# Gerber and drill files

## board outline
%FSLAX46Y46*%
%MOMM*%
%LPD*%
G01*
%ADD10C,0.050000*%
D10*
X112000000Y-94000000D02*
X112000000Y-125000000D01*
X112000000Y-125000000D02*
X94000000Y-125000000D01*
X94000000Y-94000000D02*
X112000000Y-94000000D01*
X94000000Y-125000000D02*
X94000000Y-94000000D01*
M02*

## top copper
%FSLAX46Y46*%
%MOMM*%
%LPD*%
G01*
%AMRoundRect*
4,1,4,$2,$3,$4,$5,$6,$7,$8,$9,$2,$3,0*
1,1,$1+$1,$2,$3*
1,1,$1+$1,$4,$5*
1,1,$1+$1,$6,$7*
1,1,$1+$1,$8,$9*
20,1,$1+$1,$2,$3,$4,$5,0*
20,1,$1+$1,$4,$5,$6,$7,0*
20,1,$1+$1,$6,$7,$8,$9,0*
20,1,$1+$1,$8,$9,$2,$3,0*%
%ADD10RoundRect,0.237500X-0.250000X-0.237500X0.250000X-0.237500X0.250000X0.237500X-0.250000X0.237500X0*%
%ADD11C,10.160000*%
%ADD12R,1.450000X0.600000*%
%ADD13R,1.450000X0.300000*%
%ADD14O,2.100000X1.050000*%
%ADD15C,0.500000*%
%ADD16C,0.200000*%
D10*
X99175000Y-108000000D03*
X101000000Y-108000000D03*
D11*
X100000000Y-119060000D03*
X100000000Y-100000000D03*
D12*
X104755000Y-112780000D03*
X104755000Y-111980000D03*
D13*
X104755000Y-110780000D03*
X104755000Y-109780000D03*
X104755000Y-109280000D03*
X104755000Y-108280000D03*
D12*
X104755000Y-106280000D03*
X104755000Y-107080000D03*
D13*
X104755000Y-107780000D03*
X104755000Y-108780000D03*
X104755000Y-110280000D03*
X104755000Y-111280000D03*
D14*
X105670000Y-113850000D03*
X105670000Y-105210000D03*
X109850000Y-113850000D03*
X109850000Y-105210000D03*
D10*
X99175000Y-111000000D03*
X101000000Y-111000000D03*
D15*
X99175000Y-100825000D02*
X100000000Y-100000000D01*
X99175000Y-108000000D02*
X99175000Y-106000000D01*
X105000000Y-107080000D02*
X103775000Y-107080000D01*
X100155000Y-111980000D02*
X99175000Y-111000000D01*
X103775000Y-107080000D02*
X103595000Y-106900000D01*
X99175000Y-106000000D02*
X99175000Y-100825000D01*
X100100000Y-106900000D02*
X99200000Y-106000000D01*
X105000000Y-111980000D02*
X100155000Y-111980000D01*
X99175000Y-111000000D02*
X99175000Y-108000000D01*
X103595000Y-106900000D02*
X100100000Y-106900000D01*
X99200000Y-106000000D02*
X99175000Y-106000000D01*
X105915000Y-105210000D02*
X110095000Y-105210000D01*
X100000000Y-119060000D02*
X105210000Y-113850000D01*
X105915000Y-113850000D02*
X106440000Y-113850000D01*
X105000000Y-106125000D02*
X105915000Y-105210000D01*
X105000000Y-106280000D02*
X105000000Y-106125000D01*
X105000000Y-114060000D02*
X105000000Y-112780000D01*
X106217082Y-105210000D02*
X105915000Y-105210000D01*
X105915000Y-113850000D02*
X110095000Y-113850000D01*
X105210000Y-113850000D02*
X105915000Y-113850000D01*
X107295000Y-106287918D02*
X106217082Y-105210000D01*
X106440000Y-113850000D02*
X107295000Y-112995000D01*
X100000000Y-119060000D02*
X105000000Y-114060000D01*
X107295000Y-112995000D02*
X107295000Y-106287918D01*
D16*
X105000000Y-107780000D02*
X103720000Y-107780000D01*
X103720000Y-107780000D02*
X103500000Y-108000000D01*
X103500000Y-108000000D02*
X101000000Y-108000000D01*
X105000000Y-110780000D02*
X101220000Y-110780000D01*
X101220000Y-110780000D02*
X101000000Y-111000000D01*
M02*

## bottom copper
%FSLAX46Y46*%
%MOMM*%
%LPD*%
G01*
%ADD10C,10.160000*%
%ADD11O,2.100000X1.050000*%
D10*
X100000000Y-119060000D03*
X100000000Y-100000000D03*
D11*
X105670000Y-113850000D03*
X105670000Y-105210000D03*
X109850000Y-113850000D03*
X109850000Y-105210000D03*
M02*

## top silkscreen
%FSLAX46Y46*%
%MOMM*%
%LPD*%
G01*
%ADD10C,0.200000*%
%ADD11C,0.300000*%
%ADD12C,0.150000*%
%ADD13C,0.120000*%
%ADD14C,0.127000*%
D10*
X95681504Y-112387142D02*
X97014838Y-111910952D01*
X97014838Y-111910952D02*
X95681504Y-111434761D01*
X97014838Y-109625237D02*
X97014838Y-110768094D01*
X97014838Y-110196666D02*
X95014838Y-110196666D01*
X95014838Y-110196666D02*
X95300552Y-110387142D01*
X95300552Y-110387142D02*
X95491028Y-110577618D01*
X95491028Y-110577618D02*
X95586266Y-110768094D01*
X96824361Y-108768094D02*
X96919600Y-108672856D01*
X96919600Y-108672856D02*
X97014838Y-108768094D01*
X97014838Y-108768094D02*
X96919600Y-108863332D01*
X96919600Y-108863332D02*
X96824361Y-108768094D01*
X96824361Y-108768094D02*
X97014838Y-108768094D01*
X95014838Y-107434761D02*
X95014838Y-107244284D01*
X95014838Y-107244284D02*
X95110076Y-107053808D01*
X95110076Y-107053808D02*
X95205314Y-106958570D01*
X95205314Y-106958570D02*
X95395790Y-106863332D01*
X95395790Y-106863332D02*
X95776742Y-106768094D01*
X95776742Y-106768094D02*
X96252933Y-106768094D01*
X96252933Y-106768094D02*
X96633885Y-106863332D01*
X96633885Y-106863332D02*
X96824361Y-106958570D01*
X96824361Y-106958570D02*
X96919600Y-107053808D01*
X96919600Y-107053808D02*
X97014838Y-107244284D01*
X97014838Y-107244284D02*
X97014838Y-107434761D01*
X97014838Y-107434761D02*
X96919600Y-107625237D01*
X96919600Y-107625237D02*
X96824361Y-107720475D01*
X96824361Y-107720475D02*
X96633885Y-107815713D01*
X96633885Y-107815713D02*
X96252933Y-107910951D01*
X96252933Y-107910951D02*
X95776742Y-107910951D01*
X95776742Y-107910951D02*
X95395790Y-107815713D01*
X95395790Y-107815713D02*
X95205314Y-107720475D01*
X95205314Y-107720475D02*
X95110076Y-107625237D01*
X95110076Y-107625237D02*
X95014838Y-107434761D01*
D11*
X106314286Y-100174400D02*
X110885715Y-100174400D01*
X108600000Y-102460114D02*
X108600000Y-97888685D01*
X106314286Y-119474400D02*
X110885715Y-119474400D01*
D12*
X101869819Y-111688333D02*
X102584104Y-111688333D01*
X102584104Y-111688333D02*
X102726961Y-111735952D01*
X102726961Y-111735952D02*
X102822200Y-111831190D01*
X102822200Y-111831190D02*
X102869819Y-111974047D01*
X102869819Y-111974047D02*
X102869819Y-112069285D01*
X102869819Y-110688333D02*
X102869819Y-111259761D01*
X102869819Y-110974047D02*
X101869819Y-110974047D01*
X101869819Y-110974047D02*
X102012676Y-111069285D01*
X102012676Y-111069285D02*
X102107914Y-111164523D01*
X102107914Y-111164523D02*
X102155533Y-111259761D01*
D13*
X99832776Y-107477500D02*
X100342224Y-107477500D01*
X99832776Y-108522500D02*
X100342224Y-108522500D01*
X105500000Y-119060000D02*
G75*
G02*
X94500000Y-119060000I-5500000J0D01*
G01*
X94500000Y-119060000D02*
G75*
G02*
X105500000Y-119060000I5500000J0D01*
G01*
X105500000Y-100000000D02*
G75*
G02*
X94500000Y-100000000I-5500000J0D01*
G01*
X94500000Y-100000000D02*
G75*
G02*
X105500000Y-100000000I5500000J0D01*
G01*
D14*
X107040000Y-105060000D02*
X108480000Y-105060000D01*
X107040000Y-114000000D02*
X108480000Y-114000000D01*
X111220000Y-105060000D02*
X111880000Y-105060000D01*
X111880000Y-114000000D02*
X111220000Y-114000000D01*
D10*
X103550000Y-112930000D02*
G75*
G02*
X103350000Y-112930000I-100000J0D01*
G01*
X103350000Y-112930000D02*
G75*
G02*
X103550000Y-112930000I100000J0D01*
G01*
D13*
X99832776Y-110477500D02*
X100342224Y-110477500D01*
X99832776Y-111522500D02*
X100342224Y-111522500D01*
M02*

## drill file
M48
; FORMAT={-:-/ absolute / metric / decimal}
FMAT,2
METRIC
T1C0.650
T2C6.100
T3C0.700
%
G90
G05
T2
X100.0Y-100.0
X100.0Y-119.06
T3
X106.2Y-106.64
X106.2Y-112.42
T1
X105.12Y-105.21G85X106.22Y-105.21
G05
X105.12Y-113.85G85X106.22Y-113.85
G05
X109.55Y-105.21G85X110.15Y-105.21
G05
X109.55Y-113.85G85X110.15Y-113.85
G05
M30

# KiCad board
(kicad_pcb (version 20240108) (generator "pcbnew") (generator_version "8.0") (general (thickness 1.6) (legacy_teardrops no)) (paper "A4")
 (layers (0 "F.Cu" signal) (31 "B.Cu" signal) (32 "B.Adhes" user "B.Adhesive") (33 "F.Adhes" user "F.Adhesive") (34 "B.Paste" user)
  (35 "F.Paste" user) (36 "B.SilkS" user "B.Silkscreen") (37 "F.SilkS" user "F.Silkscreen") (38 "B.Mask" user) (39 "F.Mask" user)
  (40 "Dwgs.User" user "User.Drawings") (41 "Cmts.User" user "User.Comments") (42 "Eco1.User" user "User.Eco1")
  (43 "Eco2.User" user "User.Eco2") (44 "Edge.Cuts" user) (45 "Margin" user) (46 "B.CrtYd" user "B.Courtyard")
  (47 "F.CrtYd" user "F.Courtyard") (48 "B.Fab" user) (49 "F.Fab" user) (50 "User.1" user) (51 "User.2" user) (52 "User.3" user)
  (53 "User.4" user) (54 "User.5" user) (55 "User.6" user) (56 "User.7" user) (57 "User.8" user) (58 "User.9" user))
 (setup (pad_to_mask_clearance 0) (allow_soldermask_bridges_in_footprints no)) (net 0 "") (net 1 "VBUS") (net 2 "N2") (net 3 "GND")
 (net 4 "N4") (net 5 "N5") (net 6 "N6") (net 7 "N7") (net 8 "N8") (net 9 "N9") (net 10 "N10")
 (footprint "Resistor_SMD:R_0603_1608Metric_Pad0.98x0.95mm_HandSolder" (layer "F.Cu") (at 100.0875 108)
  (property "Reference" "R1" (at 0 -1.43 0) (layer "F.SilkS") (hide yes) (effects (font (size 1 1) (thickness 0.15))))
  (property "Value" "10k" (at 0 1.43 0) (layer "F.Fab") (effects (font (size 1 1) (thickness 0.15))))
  (fp_line (start -0.254724 -0.5225) (end 0.254724 -0.5225) (stroke (width 0.12) (type solid)) (layer "F.SilkS"))
  (fp_line (start -0.254724 0.5225) (end 0.254724 0.5225) (stroke (width 0.12) (type solid)) (layer "F.SilkS"))
  (pad "1" smd roundrect (at -0.9125 0) (size 0.975 0.95) (layers "F.Cu" "F.Paste" "F.Mask") (roundrect_rratio 0.25) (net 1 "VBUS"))
  (pad "2" smd roundrect (at 0.9125 0) (size 0.975 0.95) (layers "F.Cu" "F.Paste" "F.Mask") (roundrect_rratio 0.25) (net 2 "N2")))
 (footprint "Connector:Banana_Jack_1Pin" (layer "F.Cu") (at 100 119.06)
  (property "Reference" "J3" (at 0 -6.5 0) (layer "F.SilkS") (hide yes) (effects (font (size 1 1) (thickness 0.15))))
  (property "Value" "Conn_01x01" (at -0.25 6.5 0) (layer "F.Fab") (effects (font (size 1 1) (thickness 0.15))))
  (fp_circle (center 0 0) (end 5.5 0) (stroke (width 0.12) (type solid)) (fill none) (layer "F.SilkS"))
  (pad "1" thru_hole circle (at 0 0) (size 10.16 10.16) (drill 6.1) (layers "*.Cu" "*.Mask") (remove_unused_layers no) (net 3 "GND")))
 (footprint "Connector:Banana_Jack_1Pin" (layer "F.Cu") (at 100 100)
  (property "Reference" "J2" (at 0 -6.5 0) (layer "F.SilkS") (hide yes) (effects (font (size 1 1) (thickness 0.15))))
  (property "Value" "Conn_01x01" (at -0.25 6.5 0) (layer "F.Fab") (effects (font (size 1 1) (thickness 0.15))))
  (fp_circle (center 0 0) (end 5.5 0) (stroke (width 0.12) (type solid)) (fill none) (layer "F.SilkS"))
  (pad "1" thru_hole circle (at 0 0) (size 10.16 10.16) (drill 6.1) (layers "*.Cu" "*.Mask") (remove_unused_layers no) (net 1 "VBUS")))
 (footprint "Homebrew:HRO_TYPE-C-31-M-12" (layer "F.Cu") (at 107.38 109.53 90)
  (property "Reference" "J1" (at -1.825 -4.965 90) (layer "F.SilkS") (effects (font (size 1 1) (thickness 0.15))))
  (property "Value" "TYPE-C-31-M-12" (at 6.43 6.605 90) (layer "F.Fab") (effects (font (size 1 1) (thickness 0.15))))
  (fp_line (start 4.47 -0.34) (end 4.47 1.1) (stroke (width 0.127) (type solid)) (layer "F.SilkS"))
  (fp_line (start -4.47 -0.34) (end -4.47 1.1) (stroke (width 0.127) (type solid)) (layer "F.SilkS"))
  (fp_line (start 4.47 3.84) (end 4.47 4.5) (stroke (width 0.127) (type solid)) (layer "F.SilkS"))
  (fp_line (start -4.47 4.5) (end -4.47 3.84) (stroke (width 0.127) (type solid)) (layer "F.SilkS"))
  (fp_circle (center -3.4 -3.93) (end -3.3 -3.93) (stroke (width 0.2) (type solid)) (fill none) (layer "F.SilkS"))
  (pad "" np_thru_hole circle (at -2.89 -1.18 90) (size 0.7 0.7) (drill 0.7) (layers "*.Cu" "*.Mask"))
  (pad "" np_thru_hole circle (at 2.89 -1.18 90) (size 0.7 0.7) (drill 0.7) (layers "*.Cu" "*.Mask"))
  (pad "A1B12" smd rect (at -3.25 -2.625 90) (size 0.6 1.45) (layers "F.Cu" "F.Paste" "F.Mask") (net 3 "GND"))
  (pad "A4B9" smd rect (at -2.45 -2.625 90) (size 0.6 1.45) (layers "F.Cu" "F.Paste" "F.Mask") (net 1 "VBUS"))
  (pad "A5" smd rect (at -1.25 -2.625 90) (size 0.3 1.45) (layers "F.Cu" "F.Paste" "F.Mask") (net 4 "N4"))
  (pad "A6" smd rect (at -0.25 -2.625 90) (size 0.3 1.45) (layers "F.Cu" "F.Paste" "F.Mask") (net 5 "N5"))
  (pad "A7" smd rect (at 0.25 -2.625 90) (size 0.3 1.45) (layers "F.Cu" "F.Paste" "F.Mask") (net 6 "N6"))
  (pad "A8" smd rect (at 1.25 -2.625 90) (size 0.3 1.45) (layers "F.Cu" "F.Paste" "F.Mask") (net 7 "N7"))
  (pad "B1A12" smd rect (at 3.25 -2.625 90) (size 0.6 1.45) (layers "F.Cu" "F.Paste" "F.Mask") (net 3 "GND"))
  (pad "B4A9" smd rect (at 2.45 -2.625 90) (size 0.6 1.45) (layers "F.Cu" "F.Paste" "F.Mask") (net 1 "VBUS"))
  (pad "B5" smd rect (at 1.75 -2.625 90) (size 0.3 1.45) (layers "F.Cu" "F.Paste" "F.Mask") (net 2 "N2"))
  (pad "B6" smd rect (at 0.75 -2.625 90) (size 0.3 1.45) (layers "F.Cu" "F.Paste" "F.Mask") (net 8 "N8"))
  (pad "B7" smd rect (at -0.75 -2.625 90) (size 0.3 1.45) (layers "F.Cu" "F.Paste" "F.Mask") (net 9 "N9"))
  (pad "B8" smd rect (at -1.75 -2.625 90) (size 0.3 1.45) (layers "F.Cu" "F.Paste" "F.Mask") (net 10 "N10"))
  (pad "S1" thru_hole oval (at -4.32 -1.71 90) (size 1.05 2.1) (drill oval 0.65 1.75) (layers "*.Cu" "*.Mask") (remove_unused_layers no)
   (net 3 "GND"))
  (pad "S2" thru_hole oval (at 4.32 -1.71 90) (size 1.05 2.1) (drill oval 0.65 1.75) (layers "*.Cu" "*.Mask") (remove_unused_layers no)
   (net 3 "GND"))
  (pad "S3" thru_hole oval (at -4.32 2.47 90) (size 1.05 2.1) (drill oval 0.65 1.25) (layers "*.Cu" "*.Mask") (remove_unused_layers no)
   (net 3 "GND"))
  (pad "S4" thru_hole oval (at 4.32 2.47 90) (size 1.05 2.1) (drill oval 0.65 1.25) (layers "*.Cu" "*.Mask") (remove_unused_layers no)
   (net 3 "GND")))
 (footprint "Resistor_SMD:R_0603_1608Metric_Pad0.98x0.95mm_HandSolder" (layer "F.Cu") (at 100.0875 111)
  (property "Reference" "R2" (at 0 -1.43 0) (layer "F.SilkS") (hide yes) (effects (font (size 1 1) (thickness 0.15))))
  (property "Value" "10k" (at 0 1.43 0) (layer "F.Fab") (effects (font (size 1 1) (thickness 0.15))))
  (fp_line (start -0.254724 -0.5225) (end 0.254724 -0.5225) (stroke (width 0.12) (type solid)) (layer "F.SilkS"))
  (fp_line (start -0.254724 0.5225) (end 0.254724 0.5225) (stroke (width 0.12) (type solid)) (layer "F.SilkS"))
  (pad "1" smd roundrect (at -0.9125 0) (size 0.975 0.95) (layers "F.Cu" "F.Paste" "F.Mask") (roundrect_rratio 0.25) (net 1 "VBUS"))
  (pad "2" smd roundrect (at 0.9125 0) (size 0.975 0.95) (layers "F.Cu" "F.Paste" "F.Mask") (roundrect_rratio 0.25) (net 4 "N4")))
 (gr_line (start 112 94) (end 112 125) (stroke (width 0.05) (type default)) (layer "Edge.Cuts"))
 (gr_line (start 112 125) (end 94 125) (stroke (width 0.05) (type default)) (layer "Edge.Cuts"))
 (gr_line (start 94 94) (end 112 94) (stroke (width 0.05) (type default)) (layer "Edge.Cuts"))
 (gr_line (start 94 125) (end 94 94) (stroke (width 0.05) (type default)) (layer "Edge.Cuts"))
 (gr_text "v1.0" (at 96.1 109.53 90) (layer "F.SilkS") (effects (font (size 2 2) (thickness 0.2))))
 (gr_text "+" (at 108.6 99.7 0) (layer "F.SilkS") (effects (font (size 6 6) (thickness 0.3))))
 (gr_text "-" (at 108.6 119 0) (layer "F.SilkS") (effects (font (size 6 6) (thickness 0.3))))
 (segment (start 99.175 100.825) (end 100 100) (width 0.5) (layer "F.Cu") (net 1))
 (segment (start 99.175 108) (end 99.175 106) (width 0.5) (layer "F.Cu") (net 1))
 (segment (start 105 107.08) (end 103.775 107.08) (width 0.5) (layer "F.Cu") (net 1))
 (segment (start 100.155 111.98) (end 99.175 111) (width 0.5) (layer "F.Cu") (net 1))
 (segment (start 103.775 107.08) (end 103.595 106.9) (width 0.5) (layer "F.Cu") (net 1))
 (segment (start 99.175 106) (end 99.175 100.825) (width 0.5) (layer "F.Cu") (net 1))
 (segment (start 100.1 106.9) (end 99.2 106) (width 0.5) (layer "F.Cu") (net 1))
 (segment (start 105 111.98) (end 100.155 111.98) (width 0.5) (layer "F.Cu") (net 1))
 (segment (start 99.175 111) (end 99.175 108) (width 0.5) (layer "F.Cu") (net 1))
 (segment (start 103.595 106.9) (end 100.1 106.9) (width 0.5) (layer "F.Cu") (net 1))
 (segment (start 99.2 106) (end 99.175 106) (width 0.5) (layer "F.Cu") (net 1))
 (segment (start 105.915 105.21) (end 110.095 105.21) (width 0.5) (layer "F.Cu") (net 3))
 (segment (start 100 119.06) (end 105.21 113.85) (width 0.5) (layer "F.Cu") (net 3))
 (segment (start 105.915 113.85) (end 106.44 113.85) (width 0.5) (layer "F.Cu") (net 3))
 (segment (start 105 106.125) (end 105.915 105.21) (width 0.5) (layer "F.Cu") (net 3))
 (segment (start 105 106.28) (end 105 106.125) (width 0.5) (layer "F.Cu") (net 3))
 (segment (start 105 114.06) (end 105 112.78) (width 0.5) (layer "F.Cu") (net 3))
 (segment (start 106.217082 105.21) (end 105.915 105.21) (width 0.5) (layer "F.Cu") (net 3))
 (segment (start 105.915 113.85) (end 110.095 113.85) (width 0.5) (layer "F.Cu") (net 3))
 (segment (start 105.21 113.85) (end 105.915 113.85) (width 0.5) (layer "F.Cu") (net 3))
 (segment (start 107.295 106.287918) (end 106.217082 105.21) (width 0.5) (layer "F.Cu") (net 3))
 (segment (start 106.44 113.85) (end 107.295 112.995) (width 0.5) (layer "F.Cu") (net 3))
 (segment (start 100 119.06) (end 105 114.06) (width 0.5) (layer "F.Cu") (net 3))
 (segment (start 107.295 112.995) (end 107.295 106.287918) (width 0.5) (layer "F.Cu") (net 3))
 (segment (start 105 107.78) (end 103.72 107.78) (width 0.2) (layer "F.Cu") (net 2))
 (segment (start 103.72 107.78) (end 103.5 108) (width 0.2) (layer "F.Cu") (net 2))
 (segment (start 103.5 108) (end 101 108) (width 0.2) (layer "F.Cu") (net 2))
 (segment (start 105 110.78) (end 101.22 110.78) (width 0.2) (layer "F.Cu") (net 4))
 (segment (start 101.22 110.78) (end 101 111) (width 0.2) (layer "F.Cu") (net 4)))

